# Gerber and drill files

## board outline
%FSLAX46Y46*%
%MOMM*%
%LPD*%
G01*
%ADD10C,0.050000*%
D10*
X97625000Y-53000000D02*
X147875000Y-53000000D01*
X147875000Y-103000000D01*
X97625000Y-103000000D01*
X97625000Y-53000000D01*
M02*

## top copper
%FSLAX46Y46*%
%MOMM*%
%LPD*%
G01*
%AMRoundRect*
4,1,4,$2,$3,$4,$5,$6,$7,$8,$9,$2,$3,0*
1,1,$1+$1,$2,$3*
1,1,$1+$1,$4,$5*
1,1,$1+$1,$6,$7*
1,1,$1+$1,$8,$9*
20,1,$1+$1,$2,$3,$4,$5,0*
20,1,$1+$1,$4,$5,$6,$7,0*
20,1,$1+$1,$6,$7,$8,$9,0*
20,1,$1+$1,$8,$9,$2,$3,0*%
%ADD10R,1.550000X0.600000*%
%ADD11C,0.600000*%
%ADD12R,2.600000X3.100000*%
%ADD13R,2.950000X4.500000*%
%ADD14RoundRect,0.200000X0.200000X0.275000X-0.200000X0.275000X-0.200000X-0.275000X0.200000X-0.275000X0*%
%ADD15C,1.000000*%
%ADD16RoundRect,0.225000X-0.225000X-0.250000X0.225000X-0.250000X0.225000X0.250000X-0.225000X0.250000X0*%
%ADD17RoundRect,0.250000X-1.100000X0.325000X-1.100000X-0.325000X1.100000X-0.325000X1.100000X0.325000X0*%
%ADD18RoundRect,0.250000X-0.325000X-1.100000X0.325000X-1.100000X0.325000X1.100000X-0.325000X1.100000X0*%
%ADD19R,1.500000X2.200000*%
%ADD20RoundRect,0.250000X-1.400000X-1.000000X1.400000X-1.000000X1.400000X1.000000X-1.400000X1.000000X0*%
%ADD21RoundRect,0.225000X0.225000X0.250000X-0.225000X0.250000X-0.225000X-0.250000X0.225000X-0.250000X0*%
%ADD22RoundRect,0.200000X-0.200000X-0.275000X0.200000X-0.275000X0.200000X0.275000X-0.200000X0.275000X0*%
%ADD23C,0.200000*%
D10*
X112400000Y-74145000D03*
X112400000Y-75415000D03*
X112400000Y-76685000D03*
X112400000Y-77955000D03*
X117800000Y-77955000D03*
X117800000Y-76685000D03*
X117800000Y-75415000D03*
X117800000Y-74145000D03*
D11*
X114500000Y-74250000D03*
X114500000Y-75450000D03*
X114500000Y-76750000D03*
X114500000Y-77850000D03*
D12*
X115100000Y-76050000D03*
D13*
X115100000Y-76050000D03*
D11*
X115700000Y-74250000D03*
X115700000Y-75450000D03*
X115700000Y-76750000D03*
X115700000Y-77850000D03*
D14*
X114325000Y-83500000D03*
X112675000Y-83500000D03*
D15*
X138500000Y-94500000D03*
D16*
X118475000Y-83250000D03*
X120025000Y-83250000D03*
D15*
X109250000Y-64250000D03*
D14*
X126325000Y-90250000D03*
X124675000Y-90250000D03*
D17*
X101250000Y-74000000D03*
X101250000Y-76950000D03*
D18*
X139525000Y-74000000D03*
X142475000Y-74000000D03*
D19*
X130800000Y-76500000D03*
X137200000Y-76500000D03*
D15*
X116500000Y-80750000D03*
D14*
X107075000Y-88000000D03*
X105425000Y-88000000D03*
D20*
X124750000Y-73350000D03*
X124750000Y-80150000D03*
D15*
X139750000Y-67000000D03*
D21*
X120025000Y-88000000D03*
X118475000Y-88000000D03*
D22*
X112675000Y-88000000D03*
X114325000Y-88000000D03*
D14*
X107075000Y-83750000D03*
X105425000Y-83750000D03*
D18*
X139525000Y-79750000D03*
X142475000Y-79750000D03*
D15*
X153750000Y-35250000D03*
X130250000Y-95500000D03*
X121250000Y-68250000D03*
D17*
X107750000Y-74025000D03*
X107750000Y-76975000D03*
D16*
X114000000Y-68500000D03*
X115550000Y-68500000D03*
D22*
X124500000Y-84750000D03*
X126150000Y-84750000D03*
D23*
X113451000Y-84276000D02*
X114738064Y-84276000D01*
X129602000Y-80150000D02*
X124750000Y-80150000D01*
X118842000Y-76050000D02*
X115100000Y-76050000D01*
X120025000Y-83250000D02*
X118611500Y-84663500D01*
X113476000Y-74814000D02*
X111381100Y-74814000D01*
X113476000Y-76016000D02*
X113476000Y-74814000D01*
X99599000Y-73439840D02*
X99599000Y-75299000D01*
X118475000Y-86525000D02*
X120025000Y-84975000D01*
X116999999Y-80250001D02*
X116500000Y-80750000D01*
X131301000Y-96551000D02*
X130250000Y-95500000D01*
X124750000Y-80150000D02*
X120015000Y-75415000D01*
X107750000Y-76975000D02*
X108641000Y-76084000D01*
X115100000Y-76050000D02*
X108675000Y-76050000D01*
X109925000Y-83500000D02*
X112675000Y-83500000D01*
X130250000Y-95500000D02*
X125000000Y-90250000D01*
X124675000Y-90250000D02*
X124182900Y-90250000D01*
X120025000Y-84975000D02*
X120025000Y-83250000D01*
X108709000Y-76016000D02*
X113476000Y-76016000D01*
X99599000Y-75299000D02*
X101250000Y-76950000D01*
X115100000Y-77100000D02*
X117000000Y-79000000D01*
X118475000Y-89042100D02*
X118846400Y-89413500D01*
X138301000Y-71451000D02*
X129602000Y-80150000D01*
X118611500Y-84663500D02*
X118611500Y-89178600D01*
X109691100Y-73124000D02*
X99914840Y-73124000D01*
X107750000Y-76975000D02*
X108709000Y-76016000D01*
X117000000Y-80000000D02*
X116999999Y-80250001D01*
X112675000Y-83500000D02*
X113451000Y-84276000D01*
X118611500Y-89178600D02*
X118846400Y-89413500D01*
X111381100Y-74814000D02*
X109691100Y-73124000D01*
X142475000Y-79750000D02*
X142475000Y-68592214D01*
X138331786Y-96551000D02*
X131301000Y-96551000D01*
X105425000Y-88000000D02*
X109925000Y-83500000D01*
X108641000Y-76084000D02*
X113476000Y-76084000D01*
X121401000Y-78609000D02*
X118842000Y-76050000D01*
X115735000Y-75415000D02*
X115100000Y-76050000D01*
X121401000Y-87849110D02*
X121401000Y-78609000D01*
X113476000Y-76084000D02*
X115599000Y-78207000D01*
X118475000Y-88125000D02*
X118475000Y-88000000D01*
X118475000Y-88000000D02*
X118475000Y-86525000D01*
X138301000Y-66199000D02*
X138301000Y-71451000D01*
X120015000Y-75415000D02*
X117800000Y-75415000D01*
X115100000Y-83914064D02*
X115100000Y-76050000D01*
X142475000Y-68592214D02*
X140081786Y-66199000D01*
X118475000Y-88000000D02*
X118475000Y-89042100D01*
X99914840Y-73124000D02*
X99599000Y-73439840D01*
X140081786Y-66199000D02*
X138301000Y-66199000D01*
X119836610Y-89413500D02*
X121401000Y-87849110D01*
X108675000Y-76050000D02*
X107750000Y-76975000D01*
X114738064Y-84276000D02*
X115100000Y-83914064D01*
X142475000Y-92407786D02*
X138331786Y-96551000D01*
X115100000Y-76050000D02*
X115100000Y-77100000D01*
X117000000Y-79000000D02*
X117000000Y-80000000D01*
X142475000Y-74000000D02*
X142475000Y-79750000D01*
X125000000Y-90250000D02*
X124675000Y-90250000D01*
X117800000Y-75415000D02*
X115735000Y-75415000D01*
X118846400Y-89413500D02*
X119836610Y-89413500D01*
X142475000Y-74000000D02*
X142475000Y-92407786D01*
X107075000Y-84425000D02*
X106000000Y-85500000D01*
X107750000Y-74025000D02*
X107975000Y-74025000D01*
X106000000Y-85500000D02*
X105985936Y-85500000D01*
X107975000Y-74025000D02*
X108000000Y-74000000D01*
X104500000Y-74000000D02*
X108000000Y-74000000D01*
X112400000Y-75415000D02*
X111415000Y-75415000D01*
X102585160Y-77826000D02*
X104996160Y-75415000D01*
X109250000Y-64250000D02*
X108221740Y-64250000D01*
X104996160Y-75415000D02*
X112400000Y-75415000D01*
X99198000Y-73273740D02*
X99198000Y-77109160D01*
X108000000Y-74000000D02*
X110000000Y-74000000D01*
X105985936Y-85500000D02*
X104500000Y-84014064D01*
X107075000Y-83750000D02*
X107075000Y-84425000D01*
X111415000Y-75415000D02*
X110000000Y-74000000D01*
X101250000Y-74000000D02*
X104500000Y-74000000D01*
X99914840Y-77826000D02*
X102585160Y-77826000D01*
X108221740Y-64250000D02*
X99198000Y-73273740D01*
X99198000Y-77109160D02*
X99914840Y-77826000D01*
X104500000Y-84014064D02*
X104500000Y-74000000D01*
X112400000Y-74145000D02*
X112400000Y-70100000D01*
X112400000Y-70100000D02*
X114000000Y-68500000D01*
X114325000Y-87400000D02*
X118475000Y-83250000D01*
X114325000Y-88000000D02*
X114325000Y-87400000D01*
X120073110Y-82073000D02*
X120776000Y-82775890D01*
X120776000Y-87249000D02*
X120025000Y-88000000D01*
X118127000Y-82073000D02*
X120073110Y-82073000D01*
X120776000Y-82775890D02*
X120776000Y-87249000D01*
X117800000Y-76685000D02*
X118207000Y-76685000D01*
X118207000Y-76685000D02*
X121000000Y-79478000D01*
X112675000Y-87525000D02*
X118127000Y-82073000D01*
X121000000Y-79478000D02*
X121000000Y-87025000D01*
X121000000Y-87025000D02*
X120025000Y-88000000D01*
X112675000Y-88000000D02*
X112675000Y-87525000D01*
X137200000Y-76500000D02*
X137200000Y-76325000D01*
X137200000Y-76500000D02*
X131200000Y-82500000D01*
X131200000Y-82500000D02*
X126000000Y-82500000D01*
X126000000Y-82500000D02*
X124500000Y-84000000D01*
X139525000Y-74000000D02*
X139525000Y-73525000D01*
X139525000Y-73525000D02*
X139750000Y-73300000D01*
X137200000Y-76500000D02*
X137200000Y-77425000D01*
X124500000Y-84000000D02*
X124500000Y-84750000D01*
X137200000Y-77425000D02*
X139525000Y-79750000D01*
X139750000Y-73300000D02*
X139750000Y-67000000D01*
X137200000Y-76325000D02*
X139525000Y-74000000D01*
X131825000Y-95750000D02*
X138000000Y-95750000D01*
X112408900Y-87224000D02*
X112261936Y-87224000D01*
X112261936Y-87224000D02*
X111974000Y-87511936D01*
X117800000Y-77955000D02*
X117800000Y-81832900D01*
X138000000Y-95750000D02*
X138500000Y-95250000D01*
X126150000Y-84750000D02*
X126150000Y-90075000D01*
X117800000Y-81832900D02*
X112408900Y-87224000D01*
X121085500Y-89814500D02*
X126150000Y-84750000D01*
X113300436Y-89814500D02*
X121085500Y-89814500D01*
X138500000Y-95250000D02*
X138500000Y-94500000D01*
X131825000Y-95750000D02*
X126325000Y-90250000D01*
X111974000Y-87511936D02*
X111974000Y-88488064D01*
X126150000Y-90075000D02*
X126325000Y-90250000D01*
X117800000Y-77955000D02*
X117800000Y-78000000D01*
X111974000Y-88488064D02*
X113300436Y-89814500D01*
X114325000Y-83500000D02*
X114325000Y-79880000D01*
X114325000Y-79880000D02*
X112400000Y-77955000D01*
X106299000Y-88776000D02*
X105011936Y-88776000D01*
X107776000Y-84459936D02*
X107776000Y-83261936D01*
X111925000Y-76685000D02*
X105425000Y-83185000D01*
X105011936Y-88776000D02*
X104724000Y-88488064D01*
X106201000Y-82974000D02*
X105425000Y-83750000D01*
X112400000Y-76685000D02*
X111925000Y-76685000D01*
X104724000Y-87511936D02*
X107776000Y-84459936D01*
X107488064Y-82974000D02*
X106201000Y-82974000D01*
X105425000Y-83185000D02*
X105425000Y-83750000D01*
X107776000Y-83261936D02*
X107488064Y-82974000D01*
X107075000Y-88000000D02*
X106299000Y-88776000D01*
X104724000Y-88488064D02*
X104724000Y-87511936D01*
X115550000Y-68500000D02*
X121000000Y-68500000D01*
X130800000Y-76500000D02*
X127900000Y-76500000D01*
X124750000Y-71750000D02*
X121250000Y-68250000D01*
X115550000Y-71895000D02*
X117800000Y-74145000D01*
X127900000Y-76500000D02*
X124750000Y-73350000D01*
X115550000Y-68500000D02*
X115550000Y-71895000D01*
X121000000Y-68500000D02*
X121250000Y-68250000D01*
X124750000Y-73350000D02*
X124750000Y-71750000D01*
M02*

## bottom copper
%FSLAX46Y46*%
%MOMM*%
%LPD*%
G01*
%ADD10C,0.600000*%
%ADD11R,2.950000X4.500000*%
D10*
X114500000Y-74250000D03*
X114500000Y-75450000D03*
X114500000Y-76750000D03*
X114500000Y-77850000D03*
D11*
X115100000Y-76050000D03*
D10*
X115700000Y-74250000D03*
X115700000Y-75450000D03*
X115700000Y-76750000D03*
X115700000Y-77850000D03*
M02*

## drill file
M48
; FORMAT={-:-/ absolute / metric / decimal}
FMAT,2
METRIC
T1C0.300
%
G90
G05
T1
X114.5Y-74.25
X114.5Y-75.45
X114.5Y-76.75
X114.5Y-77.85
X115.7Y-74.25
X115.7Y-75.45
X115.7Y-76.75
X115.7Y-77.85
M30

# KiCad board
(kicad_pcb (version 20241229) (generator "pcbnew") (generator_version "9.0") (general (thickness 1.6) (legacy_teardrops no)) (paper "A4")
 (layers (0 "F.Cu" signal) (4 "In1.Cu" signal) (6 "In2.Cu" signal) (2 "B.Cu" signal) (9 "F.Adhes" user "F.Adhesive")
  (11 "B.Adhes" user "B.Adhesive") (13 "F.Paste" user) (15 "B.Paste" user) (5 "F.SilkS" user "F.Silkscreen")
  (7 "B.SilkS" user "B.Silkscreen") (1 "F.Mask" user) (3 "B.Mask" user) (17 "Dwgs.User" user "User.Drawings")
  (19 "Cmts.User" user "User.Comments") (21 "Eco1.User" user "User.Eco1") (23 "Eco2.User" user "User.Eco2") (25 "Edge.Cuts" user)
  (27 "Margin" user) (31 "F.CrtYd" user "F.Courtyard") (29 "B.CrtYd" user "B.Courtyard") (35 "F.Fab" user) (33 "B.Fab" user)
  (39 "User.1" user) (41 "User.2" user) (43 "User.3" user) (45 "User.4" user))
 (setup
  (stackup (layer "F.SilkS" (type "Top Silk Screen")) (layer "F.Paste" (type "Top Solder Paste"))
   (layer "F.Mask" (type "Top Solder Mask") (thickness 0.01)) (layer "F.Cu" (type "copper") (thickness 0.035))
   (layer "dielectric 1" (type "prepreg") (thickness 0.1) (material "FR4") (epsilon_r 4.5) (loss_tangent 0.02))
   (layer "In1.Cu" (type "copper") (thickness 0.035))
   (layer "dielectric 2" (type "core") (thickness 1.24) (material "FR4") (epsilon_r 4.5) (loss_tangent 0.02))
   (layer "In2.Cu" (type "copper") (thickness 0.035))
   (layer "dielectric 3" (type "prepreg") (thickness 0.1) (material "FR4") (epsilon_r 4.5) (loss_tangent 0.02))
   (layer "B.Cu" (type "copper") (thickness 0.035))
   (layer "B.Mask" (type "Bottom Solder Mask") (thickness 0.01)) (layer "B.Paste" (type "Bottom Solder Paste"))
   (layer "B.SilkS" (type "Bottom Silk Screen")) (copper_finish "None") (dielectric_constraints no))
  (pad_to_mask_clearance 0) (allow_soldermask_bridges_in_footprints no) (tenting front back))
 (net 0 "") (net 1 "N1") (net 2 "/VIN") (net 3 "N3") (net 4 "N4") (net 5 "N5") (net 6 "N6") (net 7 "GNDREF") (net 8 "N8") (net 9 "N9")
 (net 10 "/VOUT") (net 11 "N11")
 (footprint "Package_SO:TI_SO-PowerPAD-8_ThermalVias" (layer "F.Cu") (at 115.1 76.05)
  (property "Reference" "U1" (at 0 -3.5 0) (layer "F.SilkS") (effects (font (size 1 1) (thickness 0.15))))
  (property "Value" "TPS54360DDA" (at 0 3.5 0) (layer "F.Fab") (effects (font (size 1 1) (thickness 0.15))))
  (pad "1" smd rect (at -2.7 -1.905) (size 1.55 0.6) (layers "F.Cu" "F.Mask" "F.Paste") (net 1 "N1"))
  (pad "2" smd rect (at -2.7 -0.635) (size 1.55 0.6) (layers "F.Cu" "F.Mask" "F.Paste") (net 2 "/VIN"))
  (pad "3" smd rect (at -2.7 0.635) (size 1.55 0.6) (layers "F.Cu" "F.Mask" "F.Paste") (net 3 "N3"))
  (pad "4" smd rect (at -2.7 1.905) (size 1.55 0.6) (layers "F.Cu" "F.Mask" "F.Paste") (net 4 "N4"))
  (pad "5" smd rect (at 2.7 1.905) (size 1.55 0.6) (layers "F.Cu" "F.Mask" "F.Paste") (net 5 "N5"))
  (pad "6" smd rect (at 2.7 0.635) (size 1.55 0.6) (layers "F.Cu" "F.Mask" "F.Paste") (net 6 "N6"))
  (pad "7" smd rect (at 2.7 -0.635) (size 1.55 0.6) (layers "F.Cu" "F.Mask" "F.Paste") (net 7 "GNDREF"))
  (pad "8" smd rect (at 2.7 -1.905) (size 1.55 0.6) (layers "F.Cu" "F.Mask" "F.Paste") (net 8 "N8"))
  (pad "9" thru_hole circle (at -0.6 -1.8) (size 0.6 0.6) (drill 0.3) (layers "*.Cu") (remove_unused_layers no) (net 7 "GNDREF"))
  (pad "9" thru_hole circle (at -0.6 -0.6) (size 0.6 0.6) (drill 0.3) (layers "*.Cu") (remove_unused_layers no) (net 7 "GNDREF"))
  (pad "9" thru_hole circle (at -0.6 0.7) (size 0.6 0.6) (drill 0.3) (layers "*.Cu") (remove_unused_layers no) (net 7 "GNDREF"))
  (pad "9" thru_hole circle (at -0.6 1.8) (size 0.6 0.6) (drill 0.3) (layers "*.Cu") (remove_unused_layers no) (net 7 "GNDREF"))
  (pad "9" smd rect (at 0 0) (size 2.6 3.1) (layers "F.Cu" "F.Mask" "F.Paste") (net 7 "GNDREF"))
  (pad "9" smd rect (at 0 0) (size 2.95 4.5) (layers "F.Cu") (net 7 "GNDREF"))
  (pad "9" smd rect (at 0 0) (size 2.95 4.5) (layers "B.Cu") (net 7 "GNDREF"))
  (pad "9" thru_hole circle (at 0.6 -1.8) (size 0.6 0.6) (drill 0.3) (layers "*.Cu") (remove_unused_layers no) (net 7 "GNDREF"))
  (pad "9" thru_hole circle (at 0.6 -0.6) (size 0.6 0.6) (drill 0.3) (layers "*.Cu") (remove_unused_layers no) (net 7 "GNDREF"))
  (pad "9" thru_hole circle (at 0.6 0.7) (size 0.6 0.6) (drill 0.3) (layers "*.Cu") (remove_unused_layers no) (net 7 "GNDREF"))
  (pad "9" thru_hole circle (at 0.6 1.8) (size 0.6 0.6) (drill 0.3) (layers "*.Cu") (remove_unused_layers no) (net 7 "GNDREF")))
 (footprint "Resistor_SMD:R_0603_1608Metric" (layer "F.Cu") (at 113.5 83.5 180)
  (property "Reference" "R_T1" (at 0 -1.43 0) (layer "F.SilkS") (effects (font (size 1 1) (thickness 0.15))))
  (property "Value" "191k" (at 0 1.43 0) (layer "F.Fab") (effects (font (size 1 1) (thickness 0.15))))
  (pad "1" smd roundrect (at -0.825 0 180) (size 0.8 0.95) (layers "F.Cu" "F.Mask" "F.Paste") (roundrect_rratio 0.25) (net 4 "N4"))
  (pad "2" smd roundrect (at 0.825 0 180) (size 0.8 0.95) (layers "F.Cu" "F.Mask" "F.Paste") (roundrect_rratio 0.25) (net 7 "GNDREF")))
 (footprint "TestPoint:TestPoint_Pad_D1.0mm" (layer "F.Cu") (at 138.5 94.5)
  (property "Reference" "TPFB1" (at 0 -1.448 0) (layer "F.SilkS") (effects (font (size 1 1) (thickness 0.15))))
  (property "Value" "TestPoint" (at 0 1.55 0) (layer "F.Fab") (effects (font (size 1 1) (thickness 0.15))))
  (pad "1" smd circle (at 0 0) (size 1 1) (layers "F.Cu" "F.Mask") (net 5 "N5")))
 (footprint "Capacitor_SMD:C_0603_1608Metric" (layer "F.Cu") (at 119.25 83.25)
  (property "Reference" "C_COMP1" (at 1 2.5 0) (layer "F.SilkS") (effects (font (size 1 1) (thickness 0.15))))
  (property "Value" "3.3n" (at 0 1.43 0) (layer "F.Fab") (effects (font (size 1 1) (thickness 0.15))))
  (pad "1" smd roundrect (at -0.775 0) (size 0.9 0.95) (layers "F.Cu" "F.Mask" "F.Paste") (roundrect_rratio 0.25) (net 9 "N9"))
  (pad "2" smd roundrect (at 0.775 0) (size 0.9 0.95) (layers "F.Cu" "F.Mask" "F.Paste") (roundrect_rratio 0.25) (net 7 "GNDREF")))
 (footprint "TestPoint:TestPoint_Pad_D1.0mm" (layer "F.Cu") (at 109.25 64.25)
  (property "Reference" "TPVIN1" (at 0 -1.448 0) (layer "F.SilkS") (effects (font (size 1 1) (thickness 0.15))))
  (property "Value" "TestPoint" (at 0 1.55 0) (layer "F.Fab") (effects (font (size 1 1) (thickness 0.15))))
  (pad "1" smd circle (at 0 0) (size 1 1) (layers "F.Cu" "F.Mask") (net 2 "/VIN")))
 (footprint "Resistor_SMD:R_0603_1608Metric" (layer "F.Cu") (at 125.5 90.25 180)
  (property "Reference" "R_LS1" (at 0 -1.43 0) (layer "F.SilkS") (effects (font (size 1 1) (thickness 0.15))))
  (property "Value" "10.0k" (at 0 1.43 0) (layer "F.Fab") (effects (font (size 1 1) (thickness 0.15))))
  (pad "1" smd roundrect (at -0.825 0 180) (size 0.8 0.95) (layers "F.Cu" "F.Mask" "F.Paste") (roundrect_rratio 0.25) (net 5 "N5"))
  (pad "2" smd roundrect (at 0.825 0 180) (size 0.8 0.95) (layers "F.Cu" "F.Mask" "F.Paste") (roundrect_rratio 0.25) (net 7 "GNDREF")))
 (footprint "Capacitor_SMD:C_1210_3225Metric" (layer "F.Cu") (at 101.25 75.475 -90)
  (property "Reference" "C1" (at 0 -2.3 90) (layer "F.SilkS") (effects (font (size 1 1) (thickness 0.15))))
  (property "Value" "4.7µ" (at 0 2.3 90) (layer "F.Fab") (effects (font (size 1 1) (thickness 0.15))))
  (pad "1" smd roundrect (at -1.475 0 270) (size 1.15 2.7) (layers "F.Cu" "F.Mask" "F.Paste") (roundrect_rratio 0.217391) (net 2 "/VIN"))
  (pad "2" smd roundrect (at 1.475 0 270) (size 1.15 2.7) (layers "F.Cu" "F.Mask" "F.Paste") (roundrect_rratio 0.217391) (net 7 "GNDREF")))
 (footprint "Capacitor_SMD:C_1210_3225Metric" (layer "F.Cu") (at 141 74)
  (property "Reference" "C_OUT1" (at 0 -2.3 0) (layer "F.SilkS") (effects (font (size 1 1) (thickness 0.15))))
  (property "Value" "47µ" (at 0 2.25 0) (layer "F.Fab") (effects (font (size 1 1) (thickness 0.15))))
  (pad "1" smd roundrect (at -1.475 0) (size 1.15 2.7) (layers "F.Cu" "F.Mask" "F.Paste") (roundrect_rratio 0.217391) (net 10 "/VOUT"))
  (pad "2" smd roundrect (at 1.475 0) (size 1.15 2.7) (layers "F.Cu" "F.Mask" "F.Paste") (roundrect_rratio 0.217391) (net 7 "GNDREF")))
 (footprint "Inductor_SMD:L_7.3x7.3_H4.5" (layer "F.Cu") (at 134 76.5)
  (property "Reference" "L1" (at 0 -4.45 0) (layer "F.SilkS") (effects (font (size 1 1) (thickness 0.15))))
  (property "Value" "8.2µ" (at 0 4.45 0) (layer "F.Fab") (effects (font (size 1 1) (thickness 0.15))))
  (pad "1" smd rect (at -3.2 0) (size 1.5 2.2) (layers "F.Cu" "F.Mask" "F.Paste") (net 8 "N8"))
  (pad "2" smd rect (at 3.2 0) (size 1.5 2.2) (layers "F.Cu" "F.Mask" "F.Paste") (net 10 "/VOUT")))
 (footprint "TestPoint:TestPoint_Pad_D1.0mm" (layer "F.Cu") (at 116.5 80.75)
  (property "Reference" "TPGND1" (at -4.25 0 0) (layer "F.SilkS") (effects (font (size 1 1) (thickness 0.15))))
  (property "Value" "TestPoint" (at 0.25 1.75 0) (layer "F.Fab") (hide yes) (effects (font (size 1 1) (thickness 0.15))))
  (pad "1" smd circle (at 0 0) (size 1 1) (layers "F.Cu" "F.Mask") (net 7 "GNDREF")))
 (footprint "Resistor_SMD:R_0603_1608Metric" (layer "F.Cu") (at 106.25 88 180)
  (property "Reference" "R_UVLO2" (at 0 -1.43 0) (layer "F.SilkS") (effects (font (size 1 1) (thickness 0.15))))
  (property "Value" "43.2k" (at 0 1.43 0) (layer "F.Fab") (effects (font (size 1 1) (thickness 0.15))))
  (pad "1" smd roundrect (at -0.825 0 180) (size 0.8 0.95) (layers "F.Cu" "F.Mask" "F.Paste") (roundrect_rratio 0.25) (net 3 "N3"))
  (pad "2" smd roundrect (at 0.825 0 180) (size 0.8 0.95) (layers "F.Cu" "F.Mask" "F.Paste") (roundrect_rratio 0.25) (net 7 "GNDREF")))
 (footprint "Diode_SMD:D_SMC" (layer "F.Cu") (at 124.75 76.75 -90)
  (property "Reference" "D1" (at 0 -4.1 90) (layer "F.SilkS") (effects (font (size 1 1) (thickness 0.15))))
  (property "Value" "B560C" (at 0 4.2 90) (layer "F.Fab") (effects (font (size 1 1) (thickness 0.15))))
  (pad "1" smd roundrect (at -3.4 0) (size 3.3 2.5) (layers "F.Cu" "F.Mask" "F.Paste") (roundrect_rratio 0.1) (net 8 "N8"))
  (pad "2" smd roundrect (at 3.4 0) (size 3.3 2.5) (layers "F.Cu" "F.Mask" "F.Paste") (roundrect_rratio 0.1) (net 7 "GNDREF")))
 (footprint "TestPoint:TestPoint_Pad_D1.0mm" (layer "F.Cu") (at 139.75 67)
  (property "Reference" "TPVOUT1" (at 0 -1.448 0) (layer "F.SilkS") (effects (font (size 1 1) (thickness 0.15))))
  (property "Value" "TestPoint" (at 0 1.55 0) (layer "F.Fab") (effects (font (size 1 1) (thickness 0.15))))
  (pad "1" smd circle (at 0 0) (size 1 1) (layers "F.Cu" "F.Mask") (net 10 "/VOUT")))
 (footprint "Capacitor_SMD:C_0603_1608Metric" (layer "F.Cu") (at 119.25 88 180)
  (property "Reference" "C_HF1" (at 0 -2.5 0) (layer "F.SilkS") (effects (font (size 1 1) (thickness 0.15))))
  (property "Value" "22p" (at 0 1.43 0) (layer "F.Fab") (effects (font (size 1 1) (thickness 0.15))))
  (pad "1" smd roundrect (at -0.775 0 180) (size 0.9 0.95) (layers "F.Cu" "F.Mask" "F.Paste") (roundrect_rratio 0.25) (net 6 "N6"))
  (pad "2" smd roundrect (at 0.775 0 180) (size 0.9 0.95) (layers "F.Cu" "F.Mask" "F.Paste") (roundrect_rratio 0.25) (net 7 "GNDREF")))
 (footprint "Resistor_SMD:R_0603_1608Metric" (layer "F.Cu") (at 113.5 88)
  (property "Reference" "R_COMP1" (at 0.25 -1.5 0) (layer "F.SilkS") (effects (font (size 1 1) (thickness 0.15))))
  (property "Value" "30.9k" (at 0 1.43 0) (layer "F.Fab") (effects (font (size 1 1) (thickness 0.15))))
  (pad "1" smd roundrect (at -0.825 0) (size 0.8 0.95) (layers "F.Cu" "F.Mask" "F.Paste") (roundrect_rratio 0.25) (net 6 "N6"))
  (pad "2" smd roundrect (at 0.825 0) (size 0.8 0.95) (layers "F.Cu" "F.Mask" "F.Paste") (roundrect_rratio 0.25) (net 9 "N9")))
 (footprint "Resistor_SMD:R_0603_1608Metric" (layer "F.Cu") (at 106.25 83.75 180)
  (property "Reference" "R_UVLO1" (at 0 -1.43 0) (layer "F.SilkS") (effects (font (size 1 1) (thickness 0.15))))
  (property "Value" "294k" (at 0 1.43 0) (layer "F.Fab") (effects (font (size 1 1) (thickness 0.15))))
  (pad "1" smd roundrect (at -0.825 0 180) (size 0.8 0.95) (layers "F.Cu" "F.Mask" "F.Paste") (roundrect_rratio 0.25) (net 2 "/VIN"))
  (pad "2" smd roundrect (at 0.825 0 180) (size 0.8 0.95) (layers "F.Cu" "F.Mask" "F.Paste") (roundrect_rratio 0.25) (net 3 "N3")))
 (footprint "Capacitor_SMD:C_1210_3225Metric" (layer "F.Cu") (at 141 79.75)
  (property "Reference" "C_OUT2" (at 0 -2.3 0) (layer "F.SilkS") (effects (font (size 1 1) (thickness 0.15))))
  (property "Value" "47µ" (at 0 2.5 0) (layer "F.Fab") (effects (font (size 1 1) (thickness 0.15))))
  (pad "1" smd roundrect (at -1.475 0) (size 1.15 2.7) (layers "F.Cu" "F.Mask" "F.Paste") (roundrect_rratio 0.217391) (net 10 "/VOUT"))
  (pad "2" smd roundrect (at 1.475 0) (size 1.15 2.7) (layers "F.Cu" "F.Mask" "F.Paste") (roundrect_rratio 0.217391) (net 7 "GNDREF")))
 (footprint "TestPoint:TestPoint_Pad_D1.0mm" (layer "F.Cu") (at 153.75 35.25)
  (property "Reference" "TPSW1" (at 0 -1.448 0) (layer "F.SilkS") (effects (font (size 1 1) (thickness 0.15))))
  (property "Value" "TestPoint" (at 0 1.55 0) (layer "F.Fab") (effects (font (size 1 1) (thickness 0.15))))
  (pad "1" smd circle (at 0 0) (size 1 1) (layers "F.Cu" "F.Mask") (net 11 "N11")))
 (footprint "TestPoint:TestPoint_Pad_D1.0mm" (layer "F.Cu") (at 130.25 95.5)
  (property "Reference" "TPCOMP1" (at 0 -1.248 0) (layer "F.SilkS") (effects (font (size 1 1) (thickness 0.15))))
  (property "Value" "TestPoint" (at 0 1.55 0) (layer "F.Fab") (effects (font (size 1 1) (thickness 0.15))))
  (pad "1" smd circle (at 0 0) (size 1 1) (layers "F.Cu" "F.Mask") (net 7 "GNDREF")))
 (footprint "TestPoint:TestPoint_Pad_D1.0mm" (layer "F.Cu") (at 121.25 68.25)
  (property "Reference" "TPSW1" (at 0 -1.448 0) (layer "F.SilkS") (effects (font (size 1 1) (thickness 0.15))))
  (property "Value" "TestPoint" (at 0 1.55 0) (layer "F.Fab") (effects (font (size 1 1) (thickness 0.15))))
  (pad "1" smd circle (at 0 0) (size 1 1) (layers "F.Cu" "F.Mask") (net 8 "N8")))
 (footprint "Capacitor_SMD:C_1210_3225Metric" (layer "F.Cu") (at 107.75 75.5 -90)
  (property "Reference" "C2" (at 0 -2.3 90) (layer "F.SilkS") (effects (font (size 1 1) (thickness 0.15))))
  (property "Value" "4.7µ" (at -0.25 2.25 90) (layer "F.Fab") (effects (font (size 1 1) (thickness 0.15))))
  (pad "1" smd roundrect (at -1.475 0 270) (size 1.15 2.7) (layers "F.Cu" "F.Mask" "F.Paste") (roundrect_rratio 0.217391) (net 2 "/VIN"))
  (pad "2" smd roundrect (at 1.475 0 270) (size 1.15 2.7) (layers "F.Cu" "F.Mask" "F.Paste") (roundrect_rratio 0.217391) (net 7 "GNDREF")))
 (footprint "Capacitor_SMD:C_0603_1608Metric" (layer "F.Cu") (at 114.775 68.5)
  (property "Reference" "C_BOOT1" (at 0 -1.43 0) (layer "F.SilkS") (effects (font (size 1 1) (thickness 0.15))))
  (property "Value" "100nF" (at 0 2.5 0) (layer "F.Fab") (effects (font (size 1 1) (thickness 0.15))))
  (pad "1" smd roundrect (at -0.775 0) (size 0.9 0.95) (layers "F.Cu" "F.Mask" "F.Paste") (roundrect_rratio 0.25) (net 1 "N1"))
  (pad "2" smd roundrect (at 0.775 0) (size 0.9 0.95) (layers "F.Cu" "F.Mask" "F.Paste") (roundrect_rratio 0.25) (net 8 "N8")))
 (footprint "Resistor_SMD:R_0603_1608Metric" (layer "F.Cu") (at 125.325 84.75)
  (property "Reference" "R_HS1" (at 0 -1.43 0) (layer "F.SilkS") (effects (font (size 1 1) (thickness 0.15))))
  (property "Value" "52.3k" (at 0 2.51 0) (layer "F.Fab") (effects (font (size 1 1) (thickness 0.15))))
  (pad "1" smd roundrect (at -0.825 0) (size 0.8 0.95) (layers "F.Cu" "F.Mask" "F.Paste") (roundrect_rratio 0.25) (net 10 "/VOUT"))
  (pad "2" smd roundrect (at 0.825 0) (size 0.8 0.95) (layers "F.Cu" "F.Mask" "F.Paste") (roundrect_rratio 0.25) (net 5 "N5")))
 (gr_rect (start 97.625 53) (end 147.875 103) (stroke (width 0.05) (type default)) (fill no) (layer "Edge.Cuts"))
 (segment (start 113.451 84.276) (end 114.738064 84.276) (width 0.2) (layer "F.Cu") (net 7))
 (segment (start 129.602 80.15) (end 124.75 80.15) (width 0.2) (layer "F.Cu") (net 7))
 (segment (start 118.842 76.05) (end 115.1 76.05) (width 0.2) (layer "F.Cu") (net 7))
 (segment (start 120.025 83.25) (end 118.6115 84.6635) (width 0.2) (layer "F.Cu") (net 7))
 (segment (start 113.476 74.814) (end 111.3811 74.814) (width 0.2) (layer "F.Cu") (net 7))
 (segment (start 113.476 76.016) (end 113.476 74.814) (width 0.2) (layer "F.Cu") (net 7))
 (segment (start 99.599 73.43984) (end 99.599 75.299) (width 0.2) (layer "F.Cu") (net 7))
 (segment (start 118.475 86.525) (end 120.025 84.975) (width 0.2) (layer "F.Cu") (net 7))
 (segment (start 116.999999 80.250001) (end 116.5 80.75) (width 0.2) (layer "F.Cu") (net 7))
 (segment (start 131.301 96.551) (end 130.25 95.5) (width 0.2) (layer "F.Cu") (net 7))
 (segment (start 124.75 80.15) (end 120.015 75.415) (width 0.2) (layer "F.Cu") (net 7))
 (segment (start 107.75 76.975) (end 108.641 76.084) (width 0.2) (layer "F.Cu") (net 7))
 (segment (start 115.1 76.05) (end 108.675 76.05) (width 0.2) (layer "F.Cu") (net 7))
 (segment (start 109.925 83.5) (end 112.675 83.5) (width 0.2) (layer "F.Cu") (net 7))
 (segment (start 130.25 95.5) (end 125 90.25) (width 0.2) (layer "F.Cu") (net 7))
 (segment (start 124.675 90.25) (end 124.1829 90.25) (width 0.2) (layer "F.Cu") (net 7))
 (segment (start 120.025 84.975) (end 120.025 83.25) (width 0.2) (layer "F.Cu") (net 7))
 (segment (start 108.709 76.016) (end 113.476 76.016) (width 0.2) (layer "F.Cu") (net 7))
 (segment (start 99.599 75.299) (end 101.25 76.95) (width 0.2) (layer "F.Cu") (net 7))
 (segment (start 115.1 77.1) (end 117 79) (width 0.2) (layer "F.Cu") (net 7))
 (segment (start 118.475 89.0421) (end 118.8464 89.4135) (width 0.2) (layer "F.Cu") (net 7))
 (segment (start 138.301 71.451) (end 129.602 80.15) (width 0.2) (layer "F.Cu") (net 7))
 (segment (start 118.6115 84.6635) (end 118.6115 89.1786) (width 0.2) (layer "F.Cu") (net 7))
 (segment (start 109.6911 73.124) (end 99.91484 73.124) (width 0.2) (layer "F.Cu") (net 7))
 (segment (start 107.75 76.975) (end 108.709 76.016) (width 0.2) (layer "F.Cu") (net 7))
 (segment (start 117 80) (end 116.999999 80.250001) (width 0.2) (layer "F.Cu") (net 7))
 (segment (start 112.675 83.5) (end 113.451 84.276) (width 0.2) (layer "F.Cu") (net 7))
 (segment (start 118.6115 89.1786) (end 118.8464 89.4135) (width 0.2) (layer "F.Cu") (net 7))
 (segment (start 111.3811 74.814) (end 109.6911 73.124) (width 0.2) (layer "F.Cu") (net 7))
 (segment (start 142.475 79.75) (end 142.475 68.592214) (width 0.2) (layer "F.Cu") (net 7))
 (segment (start 138.331786 96.551) (end 131.301 96.551) (width 0.2) (layer "F.Cu") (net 7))
 (segment (start 105.425 88) (end 109.925 83.5) (width 0.2) (layer "F.Cu") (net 7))
 (segment (start 108.641 76.084) (end 113.476 76.084) (width 0.2) (layer "F.Cu") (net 7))
 (segment (start 121.401 78.609) (end 118.842 76.05) (width 0.2) (layer "F.Cu") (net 7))
 (segment (start 115.735 75.415) (end 115.1 76.05) (width 0.2) (layer "F.Cu") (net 7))
 (segment (start 121.401 87.84911) (end 121.401 78.609) (width 0.2) (layer "F.Cu") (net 7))
 (segment (start 113.476 76.084) (end 115.599 78.207) (width 0.2) (layer "F.Cu") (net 7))
 (segment (start 118.475 88.125) (end 118.475 88) (width 0.2) (layer "F.Cu") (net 7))
 (segment (start 118.475 88) (end 118.475 86.525) (width 0.2) (layer "F.Cu") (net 7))
 (segment (start 138.301 66.199) (end 138.301 71.451) (width 0.2) (layer "F.Cu") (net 7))
 (segment (start 120.015 75.415) (end 117.8 75.415) (width 0.2) (layer "F.Cu") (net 7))
 (segment (start 115.1 83.914064) (end 115.1 76.05) (width 0.2) (layer "F.Cu") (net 7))
 (segment (start 142.475 68.592214) (end 140.081786 66.199) (width 0.2) (layer "F.Cu") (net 7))
 (segment (start 118.475 88) (end 118.475 89.0421) (width 0.2) (layer "F.Cu") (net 7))
 (segment (start 99.91484 73.124) (end 99.599 73.43984) (width 0.2) (layer "F.Cu") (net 7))
 (segment (start 140.081786 66.199) (end 138.301 66.199) (width 0.2) (layer "F.Cu") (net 7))
 (segment (start 119.83661 89.4135) (end 121.401 87.84911) (width 0.2) (layer "F.Cu") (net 7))
 (segment (start 108.675 76.05) (end 107.75 76.975) (width 0.2) (layer "F.Cu") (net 7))
 (segment (start 114.738064 84.276) (end 115.1 83.914064) (width 0.2) (layer "F.Cu") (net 7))
 (segment (start 142.475 92.407786) (end 138.331786 96.551) (width 0.2) (layer "F.Cu") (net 7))
 (segment (start 115.1 76.05) (end 115.1 77.1) (width 0.2) (layer "F.Cu") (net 7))
 (segment (start 117 79) (end 117 80) (width 0.2) (layer "F.Cu") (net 7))
 (segment (start 142.475 74) (end 142.475 79.75) (width 0.2) (layer "F.Cu") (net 7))
 (segment (start 125 90.25) (end 124.675 90.25) (width 0.2) (layer "F.Cu") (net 7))
 (segment (start 117.8 75.415) (end 115.735 75.415) (width 0.2) (layer "F.Cu") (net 7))
 (segment (start 118.8464 89.4135) (end 119.83661 89.4135) (width 0.2) (layer "F.Cu") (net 7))
 (segment (start 142.475 74) (end 142.475 92.407786) (width 0.2) (layer "F.Cu") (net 7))
 (segment (start 107.075 84.425) (end 106 85.5) (width 0.2) (layer "F.Cu") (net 2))
 (segment (start 107.75 74.025) (end 107.975 74.025) (width 0.2) (layer "F.Cu") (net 2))
 (segment (start 106 85.5) (end 105.985936 85.5) (width 0.2) (layer "F.Cu") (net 2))
 (segment (start 107.975 74.025) (end 108 74) (width 0.2) (layer "F.Cu") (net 2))
 (segment (start 104.5 74) (end 108 74) (width 0.2) (layer "F.Cu") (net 2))
 (segment (start 112.4 75.415) (end 111.415 75.415) (width 0.2) (layer "F.Cu") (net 2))
 (segment (start 102.58516 77.826) (end 104.99616 75.415) (width 0.2) (layer "F.Cu") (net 2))
 (segment (start 109.25 64.25) (end 108.22174 64.25) (width 0.2) (layer "F.Cu") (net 2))
 (segment (start 104.99616 75.415) (end 112.4 75.415) (width 0.2) (layer "F.Cu") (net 2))
 (segment (start 99.198 73.27374) (end 99.198 77.10916) (width 0.2) (layer "F.Cu") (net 2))
 (segment (start 108 74) (end 110 74) (width 0.2) (layer "F.Cu") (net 2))
 (segment (start 105.985936 85.5) (end 104.5 84.014064) (width 0.2) (layer "F.Cu") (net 2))
 (segment (start 107.075 83.75) (end 107.075 84.425) (width 0.2) (layer "F.Cu") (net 2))
 (segment (start 111.415 75.415) (end 110 74) (width 0.2) (layer "F.Cu") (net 2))
 (segment (start 101.25 74) (end 104.5 74) (width 0.2) (layer "F.Cu") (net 2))
 (segment (start 99.91484 77.826) (end 102.58516 77.826) (width 0.2) (layer "F.Cu") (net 2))
 (segment (start 108.22174 64.25) (end 99.198 73.27374) (width 0.2) (layer "F.Cu") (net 2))
 (segment (start 99.198 77.10916) (end 99.91484 77.826) (width 0.2) (layer "F.Cu") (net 2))
 (segment (start 104.5 84.014064) (end 104.5 74) (width 0.2) (layer "F.Cu") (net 2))
 (segment (start 112.4 74.145) (end 112.4 70.1) (width 0.2) (layer "F.Cu") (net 1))
 (segment (start 112.4 70.1) (end 114 68.5) (width 0.2) (layer "F.Cu") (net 1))
 (segment (start 114.325 87.4) (end 118.475 83.25) (width 0.2) (layer "F.Cu") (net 9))
 (segment (start 114.325 88) (end 114.325 87.4) (width 0.2) (layer "F.Cu") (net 9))
 (segment (start 120.07311 82.073) (end 120.776 82.77589) (width 0.2) (layer "F.Cu") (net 6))
 (segment (start 120.776 87.249) (end 120.025 88) (width 0.2) (layer "F.Cu") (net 6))
 (segment (start 118.127 82.073) (end 120.07311 82.073) (width 0.2) (layer "F.Cu") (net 6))
 (segment (start 120.776 82.77589) (end 120.776 87.249) (width 0.2) (layer "F.Cu") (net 6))
 (segment (start 117.8 76.685) (end 118.207 76.685) (width 0.2) (layer "F.Cu") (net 6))
 (segment (start 118.207 76.685) (end 121 79.478) (width 0.2) (layer "F.Cu") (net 6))
 (segment (start 112.675 87.525) (end 118.127 82.073) (width 0.2) (layer "F.Cu") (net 6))
 (segment (start 121 79.478) (end 121 87.025) (width 0.2) (layer "F.Cu") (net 6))
 (segment (start 121 87.025) (end 120.025 88) (width 0.2) (layer "F.Cu") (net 6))
 (segment (start 112.675 88) (end 112.675 87.525) (width 0.2) (layer "F.Cu") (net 6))
 (segment (start 137.2 76.5) (end 137.2 76.325) (width 0.2) (layer "F.Cu") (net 10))
 (segment (start 137.2 76.5) (end 131.2 82.5) (width 0.2) (layer "F.Cu") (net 10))
 (segment (start 131.2 82.5) (end 126 82.5) (width 0.2) (layer "F.Cu") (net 10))
 (segment (start 126 82.5) (end 124.5 84) (width 0.2) (layer "F.Cu") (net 10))
 (segment (start 139.525 74) (end 139.525 73.525) (width 0.2) (layer "F.Cu") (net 10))
 (segment (start 139.525 73.525) (end 139.75 73.3) (width 0.2) (layer "F.Cu") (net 10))
 (segment (start 137.2 76.5) (end 137.2 77.425) (width 0.2) (layer "F.Cu") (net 10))
 (segment (start 124.5 84) (end 124.5 84.75) (width 0.2) (layer "F.Cu") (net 10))
 (segment (start 137.2 77.425) (end 139.525 79.75) (width 0.2) (layer "F.Cu") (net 10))
 (segment (start 139.75 73.3) (end 139.75 67) (width 0.2) (layer "F.Cu") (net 10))
 (segment (start 137.2 76.325) (end 139.525 74) (width 0.2) (layer "F.Cu") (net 10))
 (segment (start 131.825 95.75) (end 138 95.75) (width 0.2) (layer "F.Cu") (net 5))
 (segment (start 112.4089 87.224) (end 112.261936 87.224) (width 0.2) (layer "F.Cu") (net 5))
 (segment (start 112.261936 87.224) (end 111.974 87.511936) (width 0.2) (layer "F.Cu") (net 5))
 (segment (start 117.8 77.955) (end 117.8 81.8329) (width 0.2) (layer "F.Cu") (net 5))
 (segment (start 138 95.75) (end 138.5 95.25) (width 0.2) (layer "F.Cu") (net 5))
 (segment (start 126.15 84.75) (end 126.15 90.075) (width 0.2) (layer "F.Cu") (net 5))
 (segment (start 117.8 81.8329) (end 112.4089 87.224) (width 0.2) (layer "F.Cu") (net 5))
 (segment (start 121.0855 89.8145) (end 126.15 84.75) (width 0.2) (layer "F.Cu") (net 5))
 (segment (start 113.300436 89.8145) (end 121.0855 89.8145) (width 0.2) (layer "F.Cu") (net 5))
 (segment (start 138.5 95.25) (end 138.5 94.5) (width 0.2) (layer "F.Cu") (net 5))
 (segment (start 131.825 95.75) (end 126.325 90.25) (width 0.2) (layer "F.Cu") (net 5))
 (segment (start 111.974 87.511936) (end 111.974 88.488064) (width 0.2) (layer "F.Cu") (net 5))
 (segment (start 126.15 90.075) (end 126.325 90.25) (width 0.2) (layer "F.Cu") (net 5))
 (segment (start 117.8 77.955) (end 117.8 78) (width 0.2) (layer "F.Cu") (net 5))
 (segment (start 111.974 88.488064) (end 113.300436 89.8145) (width 0.2) (layer "F.Cu") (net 5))
 (segment (start 114.325 83.5) (end 114.325 79.88) (width 0.2) (layer "F.Cu") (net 4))
 (segment (start 114.325 79.88) (end 112.4 77.955) (width 0.2) (layer "F.Cu") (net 4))
 (segment (start 106.299 88.776) (end 105.011936 88.776) (width 0.2) (layer "F.Cu") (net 3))
 (segment (start 107.776 84.459936) (end 107.776 83.261936) (width 0.2) (layer "F.Cu") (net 3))
 (segment (start 111.925 76.685) (end 105.425 83.185) (width 0.2) (layer "F.Cu") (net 3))
 (segment (start 105.011936 88.776) (end 104.724 88.488064) (width 0.2) (layer "F.Cu") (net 3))
 (segment (start 106.201 82.974) (end 105.425 83.75) (width 0.2) (layer "F.Cu") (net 3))
 (segment (start 112.4 76.685) (end 111.925 76.685) (width 0.2) (layer "F.Cu") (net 3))
 (segment (start 104.724 87.511936) (end 107.776 84.459936) (width 0.2) (layer "F.Cu") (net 3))
 (segment (start 107.488064 82.974) (end 106.201 82.974) (width 0.2) (layer "F.Cu") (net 3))
 (segment (start 105.425 83.185) (end 105.425 83.75) (width 0.2) (layer "F.Cu") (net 3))
 (segment (start 107.776 83.261936) (end 107.488064 82.974) (width 0.2) (layer "F.Cu") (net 3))
 (segment (start 107.075 88) (end 106.299 88.776) (width 0.2) (layer "F.Cu") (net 3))
 (segment (start 104.724 88.488064) (end 104.724 87.511936) (width 0.2) (layer "F.Cu") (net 3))
 (segment (start 115.55 68.5) (end 121 68.5) (width 0.2) (layer "F.Cu") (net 8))
 (segment (start 130.8 76.5) (end 127.9 76.5) (width 0.2) (layer "F.Cu") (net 8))
 (segment (start 124.75 71.75) (end 121.25 68.25) (width 0.2) (layer "F.Cu") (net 8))
 (segment (start 115.55 71.895) (end 117.8 74.145) (width 0.2) (layer "F.Cu") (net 8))
 (segment (start 127.9 76.5) (end 124.75 73.35) (width 0.2) (layer "F.Cu") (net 8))
 (segment (start 115.55 68.5) (end 115.55 71.895) (width 0.2) (layer "F.Cu") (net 8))
 (segment (start 121 68.5) (end 121.25 68.25) (width 0.2) (layer "F.Cu") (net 8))
 (segment (start 124.75 73.35) (end 124.75 71.75) (width 0.2) (layer "F.Cu") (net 8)))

